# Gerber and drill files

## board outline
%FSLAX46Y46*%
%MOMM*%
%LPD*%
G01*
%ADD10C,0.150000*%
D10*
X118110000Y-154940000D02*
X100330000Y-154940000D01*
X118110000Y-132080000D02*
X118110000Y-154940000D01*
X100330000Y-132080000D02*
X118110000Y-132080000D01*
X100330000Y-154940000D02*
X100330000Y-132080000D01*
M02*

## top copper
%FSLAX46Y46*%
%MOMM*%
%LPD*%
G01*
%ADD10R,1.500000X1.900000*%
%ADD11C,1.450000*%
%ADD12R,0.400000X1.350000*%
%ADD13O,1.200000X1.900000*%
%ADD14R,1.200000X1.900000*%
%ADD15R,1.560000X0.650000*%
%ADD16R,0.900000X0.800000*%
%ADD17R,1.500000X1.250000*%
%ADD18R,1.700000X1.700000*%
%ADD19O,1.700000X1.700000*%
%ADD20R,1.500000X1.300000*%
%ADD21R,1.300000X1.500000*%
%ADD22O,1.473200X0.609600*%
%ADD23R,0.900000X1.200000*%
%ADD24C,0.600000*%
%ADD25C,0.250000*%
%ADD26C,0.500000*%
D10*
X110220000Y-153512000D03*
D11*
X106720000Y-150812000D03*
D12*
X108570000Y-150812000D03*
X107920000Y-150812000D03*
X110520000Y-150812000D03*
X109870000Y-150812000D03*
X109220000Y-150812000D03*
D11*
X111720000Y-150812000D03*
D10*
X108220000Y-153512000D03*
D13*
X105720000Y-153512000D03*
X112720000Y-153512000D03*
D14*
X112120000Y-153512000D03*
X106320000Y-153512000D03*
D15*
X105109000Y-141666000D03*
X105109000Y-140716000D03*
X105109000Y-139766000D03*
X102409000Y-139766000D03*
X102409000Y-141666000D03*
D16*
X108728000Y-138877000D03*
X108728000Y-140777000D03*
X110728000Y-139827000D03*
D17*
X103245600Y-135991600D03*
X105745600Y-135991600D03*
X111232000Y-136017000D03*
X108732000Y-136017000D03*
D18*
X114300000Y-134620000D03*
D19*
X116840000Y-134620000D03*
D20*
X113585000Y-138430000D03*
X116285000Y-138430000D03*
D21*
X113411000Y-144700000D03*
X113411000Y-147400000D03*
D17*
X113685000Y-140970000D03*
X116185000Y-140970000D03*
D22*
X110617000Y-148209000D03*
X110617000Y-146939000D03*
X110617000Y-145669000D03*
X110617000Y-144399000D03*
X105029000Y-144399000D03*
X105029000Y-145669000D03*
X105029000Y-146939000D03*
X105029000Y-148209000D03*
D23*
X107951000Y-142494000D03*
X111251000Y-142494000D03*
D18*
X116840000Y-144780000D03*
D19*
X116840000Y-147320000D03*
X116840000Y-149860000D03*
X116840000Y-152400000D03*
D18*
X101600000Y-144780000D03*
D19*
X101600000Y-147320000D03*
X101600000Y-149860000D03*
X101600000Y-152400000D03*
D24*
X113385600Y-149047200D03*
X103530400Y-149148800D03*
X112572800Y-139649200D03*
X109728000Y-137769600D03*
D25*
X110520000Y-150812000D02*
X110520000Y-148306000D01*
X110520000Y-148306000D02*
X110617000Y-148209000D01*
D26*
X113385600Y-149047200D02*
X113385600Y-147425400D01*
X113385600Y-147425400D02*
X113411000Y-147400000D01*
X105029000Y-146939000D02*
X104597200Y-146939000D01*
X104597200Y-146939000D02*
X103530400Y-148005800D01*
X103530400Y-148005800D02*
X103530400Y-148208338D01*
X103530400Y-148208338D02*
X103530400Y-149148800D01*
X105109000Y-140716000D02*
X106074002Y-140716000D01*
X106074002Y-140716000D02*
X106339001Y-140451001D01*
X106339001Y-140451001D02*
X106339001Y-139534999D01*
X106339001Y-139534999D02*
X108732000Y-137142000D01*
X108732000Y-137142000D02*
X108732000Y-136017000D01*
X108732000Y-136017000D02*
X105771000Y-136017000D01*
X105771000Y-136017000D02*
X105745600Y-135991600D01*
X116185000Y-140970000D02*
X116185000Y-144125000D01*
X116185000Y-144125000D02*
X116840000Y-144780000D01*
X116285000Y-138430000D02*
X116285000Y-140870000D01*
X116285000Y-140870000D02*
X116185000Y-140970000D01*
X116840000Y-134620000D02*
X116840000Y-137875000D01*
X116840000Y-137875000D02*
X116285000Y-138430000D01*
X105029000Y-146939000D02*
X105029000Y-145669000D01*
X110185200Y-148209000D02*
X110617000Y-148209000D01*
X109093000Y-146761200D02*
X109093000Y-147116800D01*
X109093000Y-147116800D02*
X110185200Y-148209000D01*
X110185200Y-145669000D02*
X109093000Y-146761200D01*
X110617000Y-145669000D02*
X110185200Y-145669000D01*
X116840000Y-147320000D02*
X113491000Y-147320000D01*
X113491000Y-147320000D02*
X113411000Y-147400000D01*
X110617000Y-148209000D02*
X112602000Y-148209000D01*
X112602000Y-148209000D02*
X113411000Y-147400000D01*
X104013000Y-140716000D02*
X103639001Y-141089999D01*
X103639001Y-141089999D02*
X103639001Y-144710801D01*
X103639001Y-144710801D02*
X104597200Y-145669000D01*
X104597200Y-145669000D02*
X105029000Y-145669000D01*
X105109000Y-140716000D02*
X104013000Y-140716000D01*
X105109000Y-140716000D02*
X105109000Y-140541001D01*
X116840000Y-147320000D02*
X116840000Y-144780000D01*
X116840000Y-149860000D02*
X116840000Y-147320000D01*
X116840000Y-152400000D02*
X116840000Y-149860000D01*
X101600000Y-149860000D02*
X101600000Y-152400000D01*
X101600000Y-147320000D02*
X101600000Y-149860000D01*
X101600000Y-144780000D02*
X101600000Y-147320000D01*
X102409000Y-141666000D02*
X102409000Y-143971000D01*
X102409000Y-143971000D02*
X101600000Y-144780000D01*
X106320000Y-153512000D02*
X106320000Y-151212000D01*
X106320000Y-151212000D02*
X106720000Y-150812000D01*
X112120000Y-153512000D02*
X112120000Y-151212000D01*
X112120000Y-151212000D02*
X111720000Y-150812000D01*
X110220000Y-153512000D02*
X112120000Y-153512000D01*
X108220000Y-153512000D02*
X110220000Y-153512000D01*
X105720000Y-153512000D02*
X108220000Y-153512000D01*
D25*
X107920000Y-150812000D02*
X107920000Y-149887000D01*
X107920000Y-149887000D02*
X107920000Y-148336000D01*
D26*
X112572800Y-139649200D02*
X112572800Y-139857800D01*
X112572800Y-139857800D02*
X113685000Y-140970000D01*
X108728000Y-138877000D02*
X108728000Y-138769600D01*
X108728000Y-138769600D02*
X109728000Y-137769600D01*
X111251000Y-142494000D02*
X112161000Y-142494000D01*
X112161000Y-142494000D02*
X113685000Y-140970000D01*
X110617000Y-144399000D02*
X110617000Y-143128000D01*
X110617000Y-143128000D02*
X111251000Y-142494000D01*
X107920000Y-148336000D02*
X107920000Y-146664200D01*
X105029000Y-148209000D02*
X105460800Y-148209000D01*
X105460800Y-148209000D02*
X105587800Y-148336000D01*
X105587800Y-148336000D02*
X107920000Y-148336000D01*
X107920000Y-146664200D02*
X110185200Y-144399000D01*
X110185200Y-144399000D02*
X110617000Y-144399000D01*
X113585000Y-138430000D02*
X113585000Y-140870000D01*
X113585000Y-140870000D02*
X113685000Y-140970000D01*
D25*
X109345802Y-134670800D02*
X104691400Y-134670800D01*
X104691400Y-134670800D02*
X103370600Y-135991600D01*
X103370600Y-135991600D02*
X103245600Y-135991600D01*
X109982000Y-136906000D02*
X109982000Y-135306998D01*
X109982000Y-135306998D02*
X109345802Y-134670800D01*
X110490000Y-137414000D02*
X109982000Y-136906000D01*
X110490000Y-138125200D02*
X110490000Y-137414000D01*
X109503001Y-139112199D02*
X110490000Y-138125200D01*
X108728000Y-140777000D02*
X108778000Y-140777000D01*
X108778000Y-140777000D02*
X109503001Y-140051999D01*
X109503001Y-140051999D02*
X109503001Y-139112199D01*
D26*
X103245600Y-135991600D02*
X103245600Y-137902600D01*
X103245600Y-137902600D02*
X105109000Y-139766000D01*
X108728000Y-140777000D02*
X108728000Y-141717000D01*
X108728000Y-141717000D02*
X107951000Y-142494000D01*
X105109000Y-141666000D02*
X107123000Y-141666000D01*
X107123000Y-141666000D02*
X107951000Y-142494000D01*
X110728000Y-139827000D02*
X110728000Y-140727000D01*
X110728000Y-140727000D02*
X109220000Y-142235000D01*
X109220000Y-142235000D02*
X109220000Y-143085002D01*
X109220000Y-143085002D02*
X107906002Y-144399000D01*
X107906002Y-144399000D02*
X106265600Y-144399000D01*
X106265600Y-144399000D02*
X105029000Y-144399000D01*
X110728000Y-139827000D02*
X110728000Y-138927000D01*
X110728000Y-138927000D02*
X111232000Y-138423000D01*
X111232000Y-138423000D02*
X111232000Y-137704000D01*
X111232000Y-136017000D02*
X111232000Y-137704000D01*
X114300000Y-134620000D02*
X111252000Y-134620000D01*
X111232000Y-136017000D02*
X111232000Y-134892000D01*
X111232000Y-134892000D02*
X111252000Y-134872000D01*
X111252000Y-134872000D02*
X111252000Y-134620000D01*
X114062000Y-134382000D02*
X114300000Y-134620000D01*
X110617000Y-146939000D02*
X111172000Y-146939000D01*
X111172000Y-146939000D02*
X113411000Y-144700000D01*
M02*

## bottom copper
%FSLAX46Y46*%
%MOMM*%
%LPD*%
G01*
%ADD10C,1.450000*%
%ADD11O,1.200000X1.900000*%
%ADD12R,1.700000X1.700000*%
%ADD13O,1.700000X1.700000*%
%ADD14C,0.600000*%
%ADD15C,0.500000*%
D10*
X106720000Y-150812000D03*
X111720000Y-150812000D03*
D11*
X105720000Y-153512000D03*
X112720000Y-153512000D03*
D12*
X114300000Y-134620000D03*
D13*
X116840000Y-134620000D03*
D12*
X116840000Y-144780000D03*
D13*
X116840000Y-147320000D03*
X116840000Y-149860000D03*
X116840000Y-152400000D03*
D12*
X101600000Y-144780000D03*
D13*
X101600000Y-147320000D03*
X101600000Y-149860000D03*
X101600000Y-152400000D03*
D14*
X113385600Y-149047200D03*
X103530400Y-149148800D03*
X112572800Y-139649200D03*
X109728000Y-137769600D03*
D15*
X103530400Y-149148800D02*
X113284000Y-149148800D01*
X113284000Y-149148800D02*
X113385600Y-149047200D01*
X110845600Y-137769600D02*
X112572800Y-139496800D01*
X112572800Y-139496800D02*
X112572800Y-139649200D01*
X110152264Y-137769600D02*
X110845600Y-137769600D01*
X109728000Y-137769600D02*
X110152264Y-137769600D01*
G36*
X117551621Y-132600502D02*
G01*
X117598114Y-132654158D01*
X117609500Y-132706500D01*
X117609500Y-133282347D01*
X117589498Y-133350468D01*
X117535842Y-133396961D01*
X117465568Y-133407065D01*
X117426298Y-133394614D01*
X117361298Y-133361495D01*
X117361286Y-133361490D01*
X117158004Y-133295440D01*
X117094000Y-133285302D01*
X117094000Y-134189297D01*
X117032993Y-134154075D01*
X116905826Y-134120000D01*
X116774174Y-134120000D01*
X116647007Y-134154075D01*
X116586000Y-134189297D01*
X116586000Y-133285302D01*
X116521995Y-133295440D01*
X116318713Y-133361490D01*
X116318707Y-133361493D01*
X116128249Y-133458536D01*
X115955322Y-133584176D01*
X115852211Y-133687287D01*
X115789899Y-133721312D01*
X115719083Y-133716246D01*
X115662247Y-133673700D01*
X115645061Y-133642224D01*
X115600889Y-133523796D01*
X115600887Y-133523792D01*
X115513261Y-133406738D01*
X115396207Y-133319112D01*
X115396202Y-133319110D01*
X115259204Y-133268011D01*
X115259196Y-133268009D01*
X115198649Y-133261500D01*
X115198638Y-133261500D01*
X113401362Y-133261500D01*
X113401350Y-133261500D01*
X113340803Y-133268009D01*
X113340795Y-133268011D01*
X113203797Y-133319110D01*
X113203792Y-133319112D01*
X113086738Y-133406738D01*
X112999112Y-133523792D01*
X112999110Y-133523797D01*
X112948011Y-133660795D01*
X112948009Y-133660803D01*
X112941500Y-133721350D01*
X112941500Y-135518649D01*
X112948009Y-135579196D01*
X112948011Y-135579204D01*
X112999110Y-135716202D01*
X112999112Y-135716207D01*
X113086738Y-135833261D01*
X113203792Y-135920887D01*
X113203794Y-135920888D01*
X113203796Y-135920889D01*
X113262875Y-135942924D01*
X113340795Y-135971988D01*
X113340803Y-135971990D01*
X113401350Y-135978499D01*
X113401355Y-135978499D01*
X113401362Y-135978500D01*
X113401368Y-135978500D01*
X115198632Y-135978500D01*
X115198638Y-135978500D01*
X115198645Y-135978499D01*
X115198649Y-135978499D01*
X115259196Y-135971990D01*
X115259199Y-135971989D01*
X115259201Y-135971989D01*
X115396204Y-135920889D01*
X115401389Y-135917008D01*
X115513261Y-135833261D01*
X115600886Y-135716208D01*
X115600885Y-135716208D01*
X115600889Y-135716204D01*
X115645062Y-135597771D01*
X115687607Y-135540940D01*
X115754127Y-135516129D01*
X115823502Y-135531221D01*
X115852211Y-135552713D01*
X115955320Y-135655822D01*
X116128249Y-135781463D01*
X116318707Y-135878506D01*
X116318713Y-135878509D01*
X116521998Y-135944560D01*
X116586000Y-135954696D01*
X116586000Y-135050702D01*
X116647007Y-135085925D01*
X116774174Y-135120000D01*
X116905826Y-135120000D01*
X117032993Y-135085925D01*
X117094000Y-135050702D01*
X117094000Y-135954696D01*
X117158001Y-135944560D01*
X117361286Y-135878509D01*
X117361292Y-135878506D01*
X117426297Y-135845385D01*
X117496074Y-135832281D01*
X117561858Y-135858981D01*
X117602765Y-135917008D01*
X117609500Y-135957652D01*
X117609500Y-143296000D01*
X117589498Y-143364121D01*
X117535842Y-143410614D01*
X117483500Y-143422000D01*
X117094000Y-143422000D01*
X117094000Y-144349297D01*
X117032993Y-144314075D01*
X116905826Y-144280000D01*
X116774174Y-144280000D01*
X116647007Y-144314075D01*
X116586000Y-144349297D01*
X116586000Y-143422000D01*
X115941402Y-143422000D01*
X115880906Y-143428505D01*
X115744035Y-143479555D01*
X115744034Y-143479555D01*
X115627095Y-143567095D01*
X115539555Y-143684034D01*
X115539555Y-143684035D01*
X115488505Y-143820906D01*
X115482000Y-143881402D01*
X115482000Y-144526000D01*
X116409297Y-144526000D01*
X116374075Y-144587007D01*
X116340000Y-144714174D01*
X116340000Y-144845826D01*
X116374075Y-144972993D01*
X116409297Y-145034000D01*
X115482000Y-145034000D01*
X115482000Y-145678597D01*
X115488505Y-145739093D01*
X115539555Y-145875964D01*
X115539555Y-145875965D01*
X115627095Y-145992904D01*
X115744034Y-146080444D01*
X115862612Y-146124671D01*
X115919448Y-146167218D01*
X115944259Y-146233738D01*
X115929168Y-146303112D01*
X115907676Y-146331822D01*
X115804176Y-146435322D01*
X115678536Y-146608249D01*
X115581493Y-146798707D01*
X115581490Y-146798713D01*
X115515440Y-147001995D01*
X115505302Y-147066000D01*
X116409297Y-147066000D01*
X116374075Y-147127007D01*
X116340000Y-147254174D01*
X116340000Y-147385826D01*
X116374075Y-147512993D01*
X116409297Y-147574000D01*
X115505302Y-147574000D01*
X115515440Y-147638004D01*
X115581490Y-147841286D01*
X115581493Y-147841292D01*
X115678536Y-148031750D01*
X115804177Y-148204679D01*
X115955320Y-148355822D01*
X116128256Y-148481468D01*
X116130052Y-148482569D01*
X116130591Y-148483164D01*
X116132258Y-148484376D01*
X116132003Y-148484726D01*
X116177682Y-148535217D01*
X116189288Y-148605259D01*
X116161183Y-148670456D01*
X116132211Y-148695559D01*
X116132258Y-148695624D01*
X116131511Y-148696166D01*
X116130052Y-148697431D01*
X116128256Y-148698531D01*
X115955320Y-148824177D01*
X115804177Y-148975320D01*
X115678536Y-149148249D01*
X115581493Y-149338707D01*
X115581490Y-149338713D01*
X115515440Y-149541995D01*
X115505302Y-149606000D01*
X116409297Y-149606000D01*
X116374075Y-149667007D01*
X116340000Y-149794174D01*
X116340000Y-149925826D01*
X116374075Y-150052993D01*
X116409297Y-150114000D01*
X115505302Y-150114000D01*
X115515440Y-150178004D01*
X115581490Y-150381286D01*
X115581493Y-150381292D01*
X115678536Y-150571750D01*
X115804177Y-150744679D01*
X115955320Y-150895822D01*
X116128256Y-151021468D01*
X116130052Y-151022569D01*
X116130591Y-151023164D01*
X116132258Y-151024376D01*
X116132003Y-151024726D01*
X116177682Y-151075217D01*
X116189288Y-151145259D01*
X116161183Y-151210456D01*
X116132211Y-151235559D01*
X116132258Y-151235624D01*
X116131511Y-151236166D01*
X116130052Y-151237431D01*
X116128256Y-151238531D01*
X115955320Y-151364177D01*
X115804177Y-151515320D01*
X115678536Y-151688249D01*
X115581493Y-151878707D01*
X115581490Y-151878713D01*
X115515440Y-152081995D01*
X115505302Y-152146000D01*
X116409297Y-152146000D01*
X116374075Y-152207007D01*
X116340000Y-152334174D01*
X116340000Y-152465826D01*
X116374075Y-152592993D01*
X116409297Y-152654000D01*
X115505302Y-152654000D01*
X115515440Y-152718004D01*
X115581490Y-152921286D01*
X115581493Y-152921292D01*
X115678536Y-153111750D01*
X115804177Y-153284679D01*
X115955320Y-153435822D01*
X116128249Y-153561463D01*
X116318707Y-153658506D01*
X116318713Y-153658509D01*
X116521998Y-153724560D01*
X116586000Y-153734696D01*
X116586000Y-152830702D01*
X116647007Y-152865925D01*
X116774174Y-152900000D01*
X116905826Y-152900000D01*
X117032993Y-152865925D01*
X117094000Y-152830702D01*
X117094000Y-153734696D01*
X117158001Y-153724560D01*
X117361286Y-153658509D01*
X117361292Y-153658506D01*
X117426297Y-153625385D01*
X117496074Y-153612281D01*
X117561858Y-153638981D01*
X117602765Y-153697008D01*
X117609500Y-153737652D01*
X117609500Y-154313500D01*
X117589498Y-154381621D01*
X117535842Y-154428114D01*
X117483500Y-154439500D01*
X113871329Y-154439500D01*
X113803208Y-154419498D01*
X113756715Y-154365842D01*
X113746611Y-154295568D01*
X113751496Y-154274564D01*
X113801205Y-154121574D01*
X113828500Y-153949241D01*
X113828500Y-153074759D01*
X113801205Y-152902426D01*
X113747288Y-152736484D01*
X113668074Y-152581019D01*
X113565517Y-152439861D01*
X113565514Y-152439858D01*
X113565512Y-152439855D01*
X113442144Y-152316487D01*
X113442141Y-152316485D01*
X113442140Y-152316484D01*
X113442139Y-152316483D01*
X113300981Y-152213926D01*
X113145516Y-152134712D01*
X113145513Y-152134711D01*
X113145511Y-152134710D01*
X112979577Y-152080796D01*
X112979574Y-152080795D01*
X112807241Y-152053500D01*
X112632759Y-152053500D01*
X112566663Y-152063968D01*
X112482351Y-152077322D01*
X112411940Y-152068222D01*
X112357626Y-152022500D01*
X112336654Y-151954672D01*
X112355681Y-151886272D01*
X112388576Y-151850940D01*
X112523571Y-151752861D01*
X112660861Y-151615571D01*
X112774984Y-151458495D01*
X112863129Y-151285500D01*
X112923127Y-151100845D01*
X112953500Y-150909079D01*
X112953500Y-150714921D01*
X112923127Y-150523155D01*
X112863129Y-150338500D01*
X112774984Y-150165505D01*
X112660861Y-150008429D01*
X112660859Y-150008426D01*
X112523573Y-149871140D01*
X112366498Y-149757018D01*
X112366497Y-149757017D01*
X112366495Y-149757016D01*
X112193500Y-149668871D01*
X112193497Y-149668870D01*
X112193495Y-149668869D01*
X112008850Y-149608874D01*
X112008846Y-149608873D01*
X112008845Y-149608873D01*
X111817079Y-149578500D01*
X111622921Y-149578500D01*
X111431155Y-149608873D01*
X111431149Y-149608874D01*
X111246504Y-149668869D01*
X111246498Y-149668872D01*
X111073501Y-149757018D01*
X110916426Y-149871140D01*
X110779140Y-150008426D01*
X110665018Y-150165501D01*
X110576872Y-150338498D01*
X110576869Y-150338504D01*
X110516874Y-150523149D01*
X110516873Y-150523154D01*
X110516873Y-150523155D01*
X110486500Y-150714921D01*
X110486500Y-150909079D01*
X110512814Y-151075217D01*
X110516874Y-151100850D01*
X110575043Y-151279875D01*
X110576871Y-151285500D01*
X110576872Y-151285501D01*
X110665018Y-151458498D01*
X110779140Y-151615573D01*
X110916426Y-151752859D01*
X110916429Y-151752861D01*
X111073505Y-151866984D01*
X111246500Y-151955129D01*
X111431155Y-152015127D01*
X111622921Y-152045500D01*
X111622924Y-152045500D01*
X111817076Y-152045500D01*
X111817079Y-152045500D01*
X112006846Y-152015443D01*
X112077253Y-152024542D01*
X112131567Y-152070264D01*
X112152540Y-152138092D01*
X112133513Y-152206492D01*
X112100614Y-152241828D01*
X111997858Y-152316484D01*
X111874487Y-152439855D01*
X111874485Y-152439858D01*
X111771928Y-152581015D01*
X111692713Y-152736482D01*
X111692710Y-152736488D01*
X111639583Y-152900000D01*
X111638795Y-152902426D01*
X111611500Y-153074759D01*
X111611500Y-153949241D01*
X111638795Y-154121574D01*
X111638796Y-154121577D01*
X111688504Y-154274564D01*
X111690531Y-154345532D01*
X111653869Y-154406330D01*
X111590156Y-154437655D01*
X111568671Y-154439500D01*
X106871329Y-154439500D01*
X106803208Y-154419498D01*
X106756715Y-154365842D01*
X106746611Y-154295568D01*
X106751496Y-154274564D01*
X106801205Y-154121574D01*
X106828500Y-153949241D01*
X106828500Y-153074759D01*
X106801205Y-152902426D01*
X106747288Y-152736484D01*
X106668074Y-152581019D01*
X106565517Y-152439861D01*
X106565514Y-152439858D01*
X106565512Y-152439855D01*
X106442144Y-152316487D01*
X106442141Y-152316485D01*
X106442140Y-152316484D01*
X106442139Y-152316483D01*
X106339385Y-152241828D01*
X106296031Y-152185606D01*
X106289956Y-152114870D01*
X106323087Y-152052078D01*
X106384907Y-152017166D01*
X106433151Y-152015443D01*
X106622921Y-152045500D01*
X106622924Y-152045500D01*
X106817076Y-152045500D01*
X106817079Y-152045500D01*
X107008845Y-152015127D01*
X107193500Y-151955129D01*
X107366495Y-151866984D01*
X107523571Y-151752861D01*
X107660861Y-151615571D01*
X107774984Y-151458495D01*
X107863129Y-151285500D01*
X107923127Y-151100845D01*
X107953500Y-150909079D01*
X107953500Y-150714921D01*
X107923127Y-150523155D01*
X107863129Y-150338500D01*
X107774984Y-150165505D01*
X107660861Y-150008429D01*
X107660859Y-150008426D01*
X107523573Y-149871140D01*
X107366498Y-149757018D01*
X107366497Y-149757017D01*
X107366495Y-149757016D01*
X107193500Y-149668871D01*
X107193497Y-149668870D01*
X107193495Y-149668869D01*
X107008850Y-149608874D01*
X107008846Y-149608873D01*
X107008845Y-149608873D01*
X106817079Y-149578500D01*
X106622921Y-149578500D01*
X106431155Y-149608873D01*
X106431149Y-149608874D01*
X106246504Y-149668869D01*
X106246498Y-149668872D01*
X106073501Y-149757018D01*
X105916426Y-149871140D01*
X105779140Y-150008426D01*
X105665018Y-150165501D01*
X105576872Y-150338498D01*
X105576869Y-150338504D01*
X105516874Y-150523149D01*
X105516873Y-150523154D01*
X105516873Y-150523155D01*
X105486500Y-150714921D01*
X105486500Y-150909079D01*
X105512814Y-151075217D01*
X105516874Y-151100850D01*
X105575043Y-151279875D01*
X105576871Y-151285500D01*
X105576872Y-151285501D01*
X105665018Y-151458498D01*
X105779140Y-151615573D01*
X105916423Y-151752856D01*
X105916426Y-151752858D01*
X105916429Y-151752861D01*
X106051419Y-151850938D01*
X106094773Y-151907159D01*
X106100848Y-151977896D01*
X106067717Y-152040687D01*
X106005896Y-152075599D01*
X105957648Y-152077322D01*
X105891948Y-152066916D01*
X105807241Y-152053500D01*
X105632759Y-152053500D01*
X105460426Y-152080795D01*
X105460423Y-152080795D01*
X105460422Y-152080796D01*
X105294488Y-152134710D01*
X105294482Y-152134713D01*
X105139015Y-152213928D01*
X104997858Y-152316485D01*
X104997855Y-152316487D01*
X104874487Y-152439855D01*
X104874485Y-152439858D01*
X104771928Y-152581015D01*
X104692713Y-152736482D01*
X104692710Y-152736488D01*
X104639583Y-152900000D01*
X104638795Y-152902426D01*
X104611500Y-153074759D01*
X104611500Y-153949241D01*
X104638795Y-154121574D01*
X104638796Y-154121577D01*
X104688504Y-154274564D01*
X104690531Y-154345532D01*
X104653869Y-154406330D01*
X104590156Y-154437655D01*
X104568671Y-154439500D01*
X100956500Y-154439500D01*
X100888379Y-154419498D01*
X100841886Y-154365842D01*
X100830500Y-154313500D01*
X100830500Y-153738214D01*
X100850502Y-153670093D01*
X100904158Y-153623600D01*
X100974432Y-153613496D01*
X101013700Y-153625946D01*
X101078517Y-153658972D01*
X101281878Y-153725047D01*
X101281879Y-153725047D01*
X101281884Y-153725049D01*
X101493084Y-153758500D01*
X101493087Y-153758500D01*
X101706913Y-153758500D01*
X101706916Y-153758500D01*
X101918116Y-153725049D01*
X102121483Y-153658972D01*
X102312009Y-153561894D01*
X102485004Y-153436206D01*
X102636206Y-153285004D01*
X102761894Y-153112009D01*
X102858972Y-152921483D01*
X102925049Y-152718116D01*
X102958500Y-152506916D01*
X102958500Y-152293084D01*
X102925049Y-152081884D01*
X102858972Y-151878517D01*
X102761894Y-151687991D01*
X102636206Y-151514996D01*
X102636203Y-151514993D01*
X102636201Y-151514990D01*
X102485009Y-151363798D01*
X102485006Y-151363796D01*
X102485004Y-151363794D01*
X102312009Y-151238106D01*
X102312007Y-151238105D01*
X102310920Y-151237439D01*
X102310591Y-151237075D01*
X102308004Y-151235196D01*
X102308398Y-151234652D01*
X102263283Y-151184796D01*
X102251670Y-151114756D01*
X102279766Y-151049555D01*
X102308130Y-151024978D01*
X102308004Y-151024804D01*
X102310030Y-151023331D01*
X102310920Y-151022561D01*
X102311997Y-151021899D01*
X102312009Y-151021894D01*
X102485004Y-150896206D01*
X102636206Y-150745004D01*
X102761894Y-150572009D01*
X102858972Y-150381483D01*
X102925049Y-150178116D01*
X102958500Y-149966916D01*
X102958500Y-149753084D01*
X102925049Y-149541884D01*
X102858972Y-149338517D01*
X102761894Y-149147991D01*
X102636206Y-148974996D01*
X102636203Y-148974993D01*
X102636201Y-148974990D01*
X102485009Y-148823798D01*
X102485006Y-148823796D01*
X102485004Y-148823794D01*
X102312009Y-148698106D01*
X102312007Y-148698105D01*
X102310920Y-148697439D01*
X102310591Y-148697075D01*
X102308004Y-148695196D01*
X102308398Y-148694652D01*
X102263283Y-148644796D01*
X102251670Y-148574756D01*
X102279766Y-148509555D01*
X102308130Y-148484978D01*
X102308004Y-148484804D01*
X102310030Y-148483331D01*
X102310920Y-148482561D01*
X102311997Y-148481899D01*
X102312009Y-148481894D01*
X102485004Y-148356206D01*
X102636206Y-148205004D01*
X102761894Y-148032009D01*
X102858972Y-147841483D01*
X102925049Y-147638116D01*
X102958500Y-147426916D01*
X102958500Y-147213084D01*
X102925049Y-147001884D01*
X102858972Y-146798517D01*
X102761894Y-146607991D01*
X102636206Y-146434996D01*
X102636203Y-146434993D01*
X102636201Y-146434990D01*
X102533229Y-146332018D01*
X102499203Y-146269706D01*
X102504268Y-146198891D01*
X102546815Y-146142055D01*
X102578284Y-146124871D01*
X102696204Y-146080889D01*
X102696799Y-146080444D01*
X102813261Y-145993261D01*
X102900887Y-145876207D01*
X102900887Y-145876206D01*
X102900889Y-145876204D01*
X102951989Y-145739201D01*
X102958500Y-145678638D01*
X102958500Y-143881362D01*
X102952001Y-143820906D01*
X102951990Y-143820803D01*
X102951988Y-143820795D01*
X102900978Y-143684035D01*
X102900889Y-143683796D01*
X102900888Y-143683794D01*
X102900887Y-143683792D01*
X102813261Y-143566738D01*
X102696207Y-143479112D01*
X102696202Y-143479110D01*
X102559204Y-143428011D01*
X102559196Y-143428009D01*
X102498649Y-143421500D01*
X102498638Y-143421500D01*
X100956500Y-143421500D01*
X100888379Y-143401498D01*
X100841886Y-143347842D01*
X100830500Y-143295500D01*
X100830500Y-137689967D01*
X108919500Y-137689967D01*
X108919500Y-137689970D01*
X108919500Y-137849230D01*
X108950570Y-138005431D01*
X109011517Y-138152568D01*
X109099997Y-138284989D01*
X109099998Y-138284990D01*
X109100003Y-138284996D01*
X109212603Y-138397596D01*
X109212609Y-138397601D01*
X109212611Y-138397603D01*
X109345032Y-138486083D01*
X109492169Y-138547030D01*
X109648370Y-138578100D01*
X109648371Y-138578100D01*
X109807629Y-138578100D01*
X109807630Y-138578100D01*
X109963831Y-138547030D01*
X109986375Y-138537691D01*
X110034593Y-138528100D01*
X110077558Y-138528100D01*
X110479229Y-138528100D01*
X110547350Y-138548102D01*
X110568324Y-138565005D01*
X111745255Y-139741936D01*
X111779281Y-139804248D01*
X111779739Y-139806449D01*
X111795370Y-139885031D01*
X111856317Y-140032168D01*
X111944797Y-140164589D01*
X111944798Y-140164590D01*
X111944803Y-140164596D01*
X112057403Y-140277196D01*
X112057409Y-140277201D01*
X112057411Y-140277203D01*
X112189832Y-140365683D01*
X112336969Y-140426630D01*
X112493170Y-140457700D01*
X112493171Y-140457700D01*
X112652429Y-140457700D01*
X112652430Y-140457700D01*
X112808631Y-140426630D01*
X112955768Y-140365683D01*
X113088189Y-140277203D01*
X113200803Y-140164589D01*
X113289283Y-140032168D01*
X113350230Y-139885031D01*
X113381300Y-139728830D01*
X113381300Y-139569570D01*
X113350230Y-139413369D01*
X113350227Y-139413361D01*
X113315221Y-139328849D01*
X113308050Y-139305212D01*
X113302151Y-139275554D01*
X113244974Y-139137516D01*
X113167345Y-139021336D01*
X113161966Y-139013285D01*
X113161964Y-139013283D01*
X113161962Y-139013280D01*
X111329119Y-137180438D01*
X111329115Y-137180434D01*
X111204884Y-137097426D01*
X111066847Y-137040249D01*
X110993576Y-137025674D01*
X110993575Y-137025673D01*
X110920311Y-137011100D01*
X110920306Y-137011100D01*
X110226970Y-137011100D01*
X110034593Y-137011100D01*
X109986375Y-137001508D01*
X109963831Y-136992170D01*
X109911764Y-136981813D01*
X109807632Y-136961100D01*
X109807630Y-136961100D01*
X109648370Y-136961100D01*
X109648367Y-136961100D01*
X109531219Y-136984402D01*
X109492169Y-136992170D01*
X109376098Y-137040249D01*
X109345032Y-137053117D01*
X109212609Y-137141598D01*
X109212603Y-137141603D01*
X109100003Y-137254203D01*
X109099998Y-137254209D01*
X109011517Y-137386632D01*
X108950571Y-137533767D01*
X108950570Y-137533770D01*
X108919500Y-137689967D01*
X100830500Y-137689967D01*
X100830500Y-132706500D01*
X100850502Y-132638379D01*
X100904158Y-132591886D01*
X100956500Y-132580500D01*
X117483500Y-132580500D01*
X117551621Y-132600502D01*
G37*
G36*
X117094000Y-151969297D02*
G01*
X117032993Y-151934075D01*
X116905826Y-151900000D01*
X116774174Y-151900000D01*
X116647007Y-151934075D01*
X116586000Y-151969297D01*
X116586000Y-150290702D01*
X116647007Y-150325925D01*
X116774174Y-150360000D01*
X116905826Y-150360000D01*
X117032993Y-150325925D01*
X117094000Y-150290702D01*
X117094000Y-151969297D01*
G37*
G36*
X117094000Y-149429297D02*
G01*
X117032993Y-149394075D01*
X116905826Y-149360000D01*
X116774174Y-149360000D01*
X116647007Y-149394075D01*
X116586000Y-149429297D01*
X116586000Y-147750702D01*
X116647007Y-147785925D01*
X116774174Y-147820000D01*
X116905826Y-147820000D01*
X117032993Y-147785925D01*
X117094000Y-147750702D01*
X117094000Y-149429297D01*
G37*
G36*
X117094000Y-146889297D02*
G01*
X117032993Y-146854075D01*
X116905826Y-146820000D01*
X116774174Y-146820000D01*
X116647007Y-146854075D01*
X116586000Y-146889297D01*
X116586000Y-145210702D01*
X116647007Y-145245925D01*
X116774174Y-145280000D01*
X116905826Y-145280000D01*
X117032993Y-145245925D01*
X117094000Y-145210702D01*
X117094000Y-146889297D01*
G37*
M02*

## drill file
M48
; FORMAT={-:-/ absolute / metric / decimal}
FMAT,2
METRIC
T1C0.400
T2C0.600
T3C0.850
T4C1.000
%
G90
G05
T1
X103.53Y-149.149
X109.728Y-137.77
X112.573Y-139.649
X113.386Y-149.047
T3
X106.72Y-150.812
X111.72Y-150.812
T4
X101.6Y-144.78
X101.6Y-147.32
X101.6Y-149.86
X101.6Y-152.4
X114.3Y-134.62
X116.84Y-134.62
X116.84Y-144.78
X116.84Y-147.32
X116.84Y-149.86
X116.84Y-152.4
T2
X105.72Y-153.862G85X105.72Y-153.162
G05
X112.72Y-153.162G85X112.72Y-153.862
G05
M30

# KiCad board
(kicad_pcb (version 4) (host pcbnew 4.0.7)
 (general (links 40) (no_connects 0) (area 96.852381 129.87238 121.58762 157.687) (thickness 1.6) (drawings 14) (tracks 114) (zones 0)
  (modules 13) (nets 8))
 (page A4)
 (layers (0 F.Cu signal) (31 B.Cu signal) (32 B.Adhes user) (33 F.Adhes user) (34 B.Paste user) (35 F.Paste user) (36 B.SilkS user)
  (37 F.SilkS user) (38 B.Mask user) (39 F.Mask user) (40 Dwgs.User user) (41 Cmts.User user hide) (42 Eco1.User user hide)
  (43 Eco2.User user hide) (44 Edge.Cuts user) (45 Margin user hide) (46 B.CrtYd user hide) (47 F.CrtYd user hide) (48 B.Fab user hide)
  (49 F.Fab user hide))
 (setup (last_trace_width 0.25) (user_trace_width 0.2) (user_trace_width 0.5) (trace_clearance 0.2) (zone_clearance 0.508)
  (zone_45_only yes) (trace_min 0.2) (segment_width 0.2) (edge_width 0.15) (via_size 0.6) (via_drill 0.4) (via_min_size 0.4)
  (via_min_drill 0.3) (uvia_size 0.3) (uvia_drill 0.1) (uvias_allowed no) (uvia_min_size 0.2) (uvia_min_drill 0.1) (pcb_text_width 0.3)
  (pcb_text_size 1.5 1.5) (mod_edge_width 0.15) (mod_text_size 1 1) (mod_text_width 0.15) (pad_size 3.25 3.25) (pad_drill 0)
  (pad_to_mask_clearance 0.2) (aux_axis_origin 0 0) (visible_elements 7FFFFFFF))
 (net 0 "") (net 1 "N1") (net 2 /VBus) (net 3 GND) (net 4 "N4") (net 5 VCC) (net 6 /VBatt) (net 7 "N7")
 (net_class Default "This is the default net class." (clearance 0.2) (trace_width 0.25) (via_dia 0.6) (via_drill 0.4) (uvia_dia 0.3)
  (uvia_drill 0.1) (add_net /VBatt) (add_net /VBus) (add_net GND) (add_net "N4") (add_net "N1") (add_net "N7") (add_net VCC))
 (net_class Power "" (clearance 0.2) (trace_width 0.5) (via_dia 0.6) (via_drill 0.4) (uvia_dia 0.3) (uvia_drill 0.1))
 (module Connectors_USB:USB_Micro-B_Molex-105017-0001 (layer F.Cu) (at 109.22 153.162)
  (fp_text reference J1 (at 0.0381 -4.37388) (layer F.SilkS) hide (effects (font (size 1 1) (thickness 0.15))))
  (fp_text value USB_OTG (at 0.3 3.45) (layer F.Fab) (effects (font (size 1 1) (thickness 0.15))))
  (pad 6 smd rect (at 1 0.35) (size 1.5 1.9) (layers F.Cu F.Paste F.Mask) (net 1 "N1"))
  (pad 6 thru_hole circle (at -2.5 -2.35) (size 1.45 1.45) (drill 0.85) (layers *.Cu *.Mask) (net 1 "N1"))
  (pad 2 smd rect (at -0.65 -2.35) (size 0.4 1.35) (layers F.Cu F.Paste F.Mask))
  (pad 1 smd rect (at -1.3 -2.35) (size 0.4 1.35) (layers F.Cu F.Paste F.Mask) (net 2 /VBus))
  (pad 5 smd rect (at 1.3 -2.35) (size 0.4 1.35) (layers F.Cu F.Paste F.Mask) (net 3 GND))
  (pad 4 smd rect (at 0.65 -2.35) (size 0.4 1.35) (layers F.Cu F.Paste F.Mask))
  (pad 3 smd rect (at 0 -2.35) (size 0.4 1.35) (layers F.Cu F.Paste F.Mask))
  (pad 6 thru_hole circle (at 2.5 -2.35) (size 1.45 1.45) (drill 0.85) (layers *.Cu *.Mask) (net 1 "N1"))
  (pad 6 smd rect (at -1 0.35) (size 1.5 1.9) (layers F.Cu F.Paste F.Mask) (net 1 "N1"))
  (pad 6 thru_hole oval (at -3.5 0.35 180) (size 1.2 1.9) (drill oval 0.6 1.3) (layers *.Cu *.Mask) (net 1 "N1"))
  (pad 6 thru_hole oval (at 3.5 0.35) (size 1.2 1.9) (drill oval 0.6 1.3) (layers *.Cu *.Mask) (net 1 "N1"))
  (pad 6 smd rect (at 2.9 0.35) (size 1.2 1.9) (layers F.Cu F.Mask) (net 1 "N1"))
  (pad 6 smd rect (at -2.9 0.35) (size 1.2 1.9) (layers F.Cu F.Mask) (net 1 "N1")))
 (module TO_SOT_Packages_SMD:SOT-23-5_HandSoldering (layer F.Cu) (at 103.759 140.716 180)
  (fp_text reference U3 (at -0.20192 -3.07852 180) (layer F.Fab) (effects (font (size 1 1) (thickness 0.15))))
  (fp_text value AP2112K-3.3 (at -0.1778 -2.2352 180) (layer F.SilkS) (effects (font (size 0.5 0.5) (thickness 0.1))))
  (pad 1 smd rect (at -1.35 -0.95 180) (size 1.56 0.65) (layers F.Cu F.Paste F.Mask) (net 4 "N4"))
  (pad 2 smd rect (at -1.35 0 180) (size 1.56 0.65) (layers F.Cu F.Paste F.Mask) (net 3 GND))
  (pad 3 smd rect (at -1.35 0.95 180) (size 1.56 0.65) (layers F.Cu F.Paste F.Mask) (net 4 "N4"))
  (pad 4 smd rect (at 1.35 0.95 180) (size 1.56 0.65) (layers F.Cu F.Paste F.Mask))
  (pad 5 smd rect (at 1.35 -0.95 180) (size 1.56 0.65) (layers F.Cu F.Paste F.Mask) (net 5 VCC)))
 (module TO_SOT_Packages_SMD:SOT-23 (layer F.Cu) (at 109.728 139.827)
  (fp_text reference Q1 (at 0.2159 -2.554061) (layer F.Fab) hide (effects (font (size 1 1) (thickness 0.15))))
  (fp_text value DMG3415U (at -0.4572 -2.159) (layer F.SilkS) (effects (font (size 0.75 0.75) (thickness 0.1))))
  (pad 1 smd rect (at -1 -0.95) (size 0.9 0.8) (layers F.Cu F.Paste F.Mask) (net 2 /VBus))
  (pad 2 smd rect (at -1 0.95) (size 0.9 0.8) (layers F.Cu F.Paste F.Mask) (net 4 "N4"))
  (pad 3 smd rect (at 1 0) (size 0.9 0.8) (layers F.Cu F.Paste F.Mask) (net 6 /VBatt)))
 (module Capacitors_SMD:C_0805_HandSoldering (layer F.Cu) (at 104.4956 135.9916)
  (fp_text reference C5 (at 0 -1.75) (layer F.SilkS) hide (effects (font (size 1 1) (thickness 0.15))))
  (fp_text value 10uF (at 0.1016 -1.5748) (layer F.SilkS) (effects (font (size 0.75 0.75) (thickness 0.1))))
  (pad 1 smd rect (at -1.25 0) (size 1.5 1.25) (layers F.Cu F.Paste F.Mask) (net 4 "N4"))
  (pad 2 smd rect (at 1.25 0) (size 1.5 1.25) (layers F.Cu F.Paste F.Mask) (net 3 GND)))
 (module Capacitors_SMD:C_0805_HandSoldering (layer F.Cu) (at 109.982 136.017 180)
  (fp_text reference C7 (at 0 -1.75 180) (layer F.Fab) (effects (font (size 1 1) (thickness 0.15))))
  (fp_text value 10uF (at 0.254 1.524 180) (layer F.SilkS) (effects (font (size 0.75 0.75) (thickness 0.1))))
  (pad 1 smd rect (at -1.25 0 180) (size 1.5 1.25) (layers F.Cu F.Paste F.Mask) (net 6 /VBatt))
  (pad 2 smd rect (at 1.25 0 180) (size 1.5 1.25) (layers F.Cu F.Paste F.Mask) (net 3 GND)))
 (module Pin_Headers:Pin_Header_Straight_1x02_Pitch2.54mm (layer F.Cu) (at 114.3 134.62 90)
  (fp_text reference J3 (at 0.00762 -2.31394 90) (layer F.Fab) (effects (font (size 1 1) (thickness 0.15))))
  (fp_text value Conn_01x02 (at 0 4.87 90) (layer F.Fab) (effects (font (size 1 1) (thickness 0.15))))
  (pad 1 thru_hole rect (at 0 0 90) (size 1.7 1.7) (drill 1) (layers *.Cu *.Mask) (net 6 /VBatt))
  (pad 2 thru_hole oval (at 0 2.54 90) (size 1.7 1.7) (drill 1) (layers *.Cu *.Mask) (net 3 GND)))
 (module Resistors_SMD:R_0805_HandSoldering (layer F.Cu) (at 114.935 138.43)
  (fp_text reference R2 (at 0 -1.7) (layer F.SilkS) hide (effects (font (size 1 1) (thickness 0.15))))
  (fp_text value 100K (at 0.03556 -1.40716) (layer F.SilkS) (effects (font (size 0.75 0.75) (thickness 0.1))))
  (pad 1 smd rect (at -1.35 0) (size 1.5 1.3) (layers F.Cu F.Paste F.Mask) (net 2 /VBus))
  (pad 2 smd rect (at 1.35 0) (size 1.5 1.3) (layers F.Cu F.Paste F.Mask) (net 3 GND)))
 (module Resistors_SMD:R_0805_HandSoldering (layer F.Cu) (at 113.411 146.05 270)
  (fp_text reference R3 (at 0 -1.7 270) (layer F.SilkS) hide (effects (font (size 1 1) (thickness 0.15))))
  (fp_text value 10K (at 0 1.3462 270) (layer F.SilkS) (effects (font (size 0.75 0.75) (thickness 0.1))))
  (pad 1 smd rect (at -1.35 0 270) (size 1.5 1.3) (layers F.Cu F.Paste F.Mask) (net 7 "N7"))
  (pad 2 smd rect (at 1.35 0 270) (size 1.5 1.3) (layers F.Cu F.Paste F.Mask) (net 3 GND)))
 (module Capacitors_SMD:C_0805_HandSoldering (layer F.Cu) (at 114.935 140.97)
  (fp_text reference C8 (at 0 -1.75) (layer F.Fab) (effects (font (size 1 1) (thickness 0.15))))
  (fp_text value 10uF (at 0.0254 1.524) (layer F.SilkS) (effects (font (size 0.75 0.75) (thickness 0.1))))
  (pad 1 smd rect (at -1.25 0) (size 1.5 1.25) (layers F.Cu F.Paste F.Mask) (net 2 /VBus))
  (pad 2 smd rect (at 1.25 0) (size 1.5 1.25) (layers F.Cu F.Paste F.Mask) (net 3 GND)))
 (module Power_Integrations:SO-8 (layer F.Cu) (at 107.823 146.304 90)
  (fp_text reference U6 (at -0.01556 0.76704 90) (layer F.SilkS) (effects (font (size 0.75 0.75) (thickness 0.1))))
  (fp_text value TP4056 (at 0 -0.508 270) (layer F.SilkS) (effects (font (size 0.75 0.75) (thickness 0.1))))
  (pad 1 smd oval (at -1.905 2.794 90) (size 0.6096 1.4732) (layers F.Cu F.Paste F.Mask) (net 3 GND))
  (pad 2 smd oval (at -0.635 2.794 90) (size 0.6096 1.4732) (layers F.Cu F.Paste F.Mask) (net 7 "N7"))
  (pad 3 smd oval (at 0.635 2.794 90) (size 0.6096 1.4732) (layers F.Cu F.Paste F.Mask) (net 3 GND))
  (pad 4 smd oval (at 1.905 2.794 90) (size 0.6096 1.4732) (layers F.Cu F.Paste F.Mask) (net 2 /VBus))
  (pad 5 smd oval (at 1.905 -2.794 90) (size 0.6096 1.4732) (layers F.Cu F.Paste F.Mask) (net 6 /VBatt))
  (pad 6 smd oval (at 0.635 -2.794 90) (size 0.6096 1.4732) (layers F.Cu F.Paste F.Mask) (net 3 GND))
  (pad 7 smd oval (at -0.635 -2.794 90) (size 0.6096 1.4732) (layers F.Cu F.Paste F.Mask) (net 3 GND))
  (pad 8 smd oval (at -1.905 -2.794 90) (size 0.6096 1.4732) (layers F.Cu F.Paste F.Mask) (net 2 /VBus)))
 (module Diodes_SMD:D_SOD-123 (layer F.Cu) (at 109.601 142.494)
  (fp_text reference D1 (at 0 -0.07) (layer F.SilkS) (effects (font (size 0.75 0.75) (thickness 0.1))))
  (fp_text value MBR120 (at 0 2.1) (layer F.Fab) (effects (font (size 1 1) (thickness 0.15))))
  (pad 1 smd rect (at -1.65 0) (size 0.9 1.2) (layers F.Cu F.Paste F.Mask) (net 4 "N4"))
  (pad 2 smd rect (at 1.65 0) (size 0.9 1.2) (layers F.Cu F.Paste F.Mask) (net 2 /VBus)))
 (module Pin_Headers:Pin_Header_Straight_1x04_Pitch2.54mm (layer F.Cu) (at 116.84 144.78)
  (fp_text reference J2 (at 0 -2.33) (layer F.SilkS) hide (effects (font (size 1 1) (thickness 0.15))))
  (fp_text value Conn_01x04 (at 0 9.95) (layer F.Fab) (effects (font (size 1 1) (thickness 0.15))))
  (pad 1 thru_hole rect (at 0 0) (size 1.7 1.7) (drill 1) (layers *.Cu *.Mask) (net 3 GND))
  (pad 2 thru_hole oval (at 0 2.54) (size 1.7 1.7) (drill 1) (layers *.Cu *.Mask) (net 3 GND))
  (pad 3 thru_hole oval (at 0 5.08) (size 1.7 1.7) (drill 1) (layers *.Cu *.Mask) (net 3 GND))
  (pad 4 thru_hole oval (at 0 7.62) (size 1.7 1.7) (drill 1) (layers *.Cu *.Mask) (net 3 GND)))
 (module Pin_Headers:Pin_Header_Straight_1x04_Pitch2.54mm (layer F.Cu) (at 101.6 144.78)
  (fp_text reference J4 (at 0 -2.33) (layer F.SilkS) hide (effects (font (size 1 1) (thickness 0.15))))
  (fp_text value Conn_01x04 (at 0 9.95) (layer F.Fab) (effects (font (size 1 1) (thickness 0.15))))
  (pad 1 thru_hole rect (at 0 0) (size 1.7 1.7) (drill 1) (layers *.Cu *.Mask) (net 5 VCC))
  (pad 2 thru_hole oval (at 0 2.54) (size 1.7 1.7) (drill 1) (layers *.Cu *.Mask) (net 5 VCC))
  (pad 3 thru_hole oval (at 0 5.08) (size 1.7 1.7) (drill 1) (layers *.Cu *.Mask) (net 5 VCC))
  (pad 4 thru_hole oval (at 0 7.62) (size 1.7 1.7) (drill 1) (layers *.Cu *.Mask) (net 5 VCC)))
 (gr_line (start 118.11 154.94) (end 100.33 154.94) (layer Edge.Cuts) (width 0.15))
 (gr_line (start 118.11 132.08) (end 118.11 154.94) (layer Edge.Cuts) (width 0.15))
 (gr_line (start 100.33 132.08) (end 118.11 132.08) (layer Edge.Cuts) (width 0.15))
 (gr_line (start 100.33 154.94) (end 100.33 132.08) (layer Edge.Cuts) (width 0.15))
 (segment (start 110.52 150.812) (end 110.52 148.306) (width 0.25) (layer F.Cu) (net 3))
 (segment (start 110.52 148.306) (end 110.617 148.209) (width 0.25) (layer F.Cu) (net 3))
 (segment (start 113.3856 149.0472) (end 113.3856 147.4254) (width 0.5) (layer F.Cu) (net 3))
 (segment (start 113.3856 147.4254) (end 113.411 147.4) (width 0.5) (layer F.Cu) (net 3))
 (segment (start 103.5304 149.1488) (end 113.284 149.1488) (width 0.5) (layer B.Cu) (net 3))
 (segment (start 113.284 149.1488) (end 113.3856 149.0472) (width 0.5) (layer B.Cu) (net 3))
 (via (at 113.3856 149.0472) (size 0.6) (drill 0.4) (layers F.Cu B.Cu) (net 3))
 (segment (start 105.029 146.939) (end 104.5972 146.939) (width 0.5) (layer F.Cu) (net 3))
 (segment (start 104.5972 146.939) (end 103.5304 148.0058) (width 0.5) (layer F.Cu) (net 3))
 (segment (start 103.5304 148.0058) (end 103.5304 148.208338) (width 0.5) (layer F.Cu) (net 3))
 (segment (start 103.5304 148.208338) (end 103.5304 149.1488) (width 0.5) (layer F.Cu) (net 3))
 (via (at 103.5304 149.1488) (size 0.6) (drill 0.4) (layers F.Cu B.Cu) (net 3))
 (segment (start 105.109 140.716) (end 106.074002 140.716) (width 0.5) (layer F.Cu) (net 3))
 (segment (start 106.074002 140.716) (end 106.339001 140.451001) (width 0.5) (layer F.Cu) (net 3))
 (segment (start 106.339001 140.451001) (end 106.339001 139.534999) (width 0.5) (layer F.Cu) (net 3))
 (segment (start 106.339001 139.534999) (end 108.732 137.142) (width 0.5) (layer F.Cu) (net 3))
 (segment (start 108.732 137.142) (end 108.732 136.017) (width 0.5) (layer F.Cu) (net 3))
 (segment (start 108.732 136.017) (end 105.771 136.017) (width 0.5) (layer F.Cu) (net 3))
 (segment (start 105.771 136.017) (end 105.7456 135.9916) (width 0.5) (layer F.Cu) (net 3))
 (segment (start 116.185 140.97) (end 116.185 144.125) (width 0.5) (layer F.Cu) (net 3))
 (segment (start 116.185 144.125) (end 116.84 144.78) (width 0.5) (layer F.Cu) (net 3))
 (segment (start 116.285 138.43) (end 116.285 140.87) (width 0.5) (layer F.Cu) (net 3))
 (segment (start 116.285 140.87) (end 116.185 140.97) (width 0.5) (layer F.Cu) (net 3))
 (segment (start 116.84 134.62) (end 116.84 137.875) (width 0.5) (layer F.Cu) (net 3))
 (segment (start 116.84 137.875) (end 116.285 138.43) (width 0.5) (layer F.Cu) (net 3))
 (segment (start 105.029 146.939) (end 105.029 145.669) (width 0.5) (layer F.Cu) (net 3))
 (segment (start 110.1852 148.209) (end 110.617 148.209) (width 0.5) (layer F.Cu) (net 3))
 (segment (start 109.093 146.7612) (end 109.093 147.1168) (width 0.5) (layer F.Cu) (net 3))
 (segment (start 109.093 147.1168) (end 110.1852 148.209) (width 0.5) (layer F.Cu) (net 3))
 (segment (start 110.1852 145.669) (end 109.093 146.7612) (width 0.5) (layer F.Cu) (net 3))
 (segment (start 110.617 145.669) (end 110.1852 145.669) (width 0.5) (layer F.Cu) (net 3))
 (segment (start 116.84 147.32) (end 113.491 147.32) (width 0.5) (layer F.Cu) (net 3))
 (segment (start 113.491 147.32) (end 113.411 147.4) (width 0.5) (layer F.Cu) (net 3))
 (segment (start 110.617 148.209) (end 112.602 148.209) (width 0.5) (layer F.Cu) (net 3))
 (segment (start 112.602 148.209) (end 113.411 147.4) (width 0.5) (layer F.Cu) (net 3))
 (segment (start 104.013 140.716) (end 103.639001 141.089999) (width 0.5) (layer F.Cu) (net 3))
 (segment (start 103.639001 141.089999) (end 103.639001 144.710801) (width 0.5) (layer F.Cu) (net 3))
 (segment (start 103.639001 144.710801) (end 104.5972 145.669) (width 0.5) (layer F.Cu) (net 3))
 (segment (start 104.5972 145.669) (end 105.029 145.669) (width 0.5) (layer F.Cu) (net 3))
 (segment (start 105.109 140.716) (end 104.013 140.716) (width 0.5) (layer F.Cu) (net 3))
 (segment (start 105.109 140.716) (end 105.109 140.541001) (width 0.5) (layer F.Cu) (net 3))
 (segment (start 116.84 147.32) (end 116.84 144.78) (width 0.5) (layer F.Cu) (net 3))
 (segment (start 116.84 149.86) (end 116.84 147.32) (width 0.5) (layer F.Cu) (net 3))
 (segment (start 116.84 152.4) (end 116.84 149.86) (width 0.5) (layer F.Cu) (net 3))
 (segment (start 101.6 149.86) (end 101.6 152.4) (width 0.5) (layer F.Cu) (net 5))
 (segment (start 101.6 147.32) (end 101.6 149.86) (width 0.5) (layer F.Cu) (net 5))
 (segment (start 101.6 144.78) (end 101.6 147.32) (width 0.5) (layer F.Cu) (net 5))
 (segment (start 102.409 141.666) (end 102.409 143.971) (width 0.5) (layer F.Cu) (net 5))
 (segment (start 102.409 143.971) (end 101.6 144.78) (width 0.5) (layer F.Cu) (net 5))
 (segment (start 106.32 153.512) (end 106.32 151.212) (width 0.5) (layer F.Cu) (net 1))
 (segment (start 106.32 151.212) (end 106.72 150.812) (width 0.5) (layer F.Cu) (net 1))
 (segment (start 112.12 153.512) (end 112.12 151.212) (width 0.5) (layer F.Cu) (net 1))
 (segment (start 112.12 151.212) (end 111.72 150.812) (width 0.5) (layer F.Cu) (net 1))
 (segment (start 110.22 153.512) (end 112.12 153.512) (width 0.5) (layer F.Cu) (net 1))
 (segment (start 108.22 153.512) (end 110.22 153.512) (width 0.5) (layer F.Cu) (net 1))
 (segment (start 105.72 153.512) (end 108.22 153.512) (width 0.5) (layer F.Cu) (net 1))
 (segment (start 107.92 150.812) (end 107.92 149.887) (width 0.25) (layer F.Cu) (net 2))
 (segment (start 107.92 149.887) (end 107.92 148.336) (width 0.25) (layer F.Cu) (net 2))
 (segment (start 112.5728 139.6492) (end 112.5728 139.8578) (width 0.5) (layer F.Cu) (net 2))
 (segment (start 112.5728 139.8578) (end 113.685 140.97) (width 0.5) (layer F.Cu) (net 2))
 (segment (start 110.8456 137.7696) (end 112.5728 139.4968) (width 0.5) (layer B.Cu) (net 2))
 (segment (start 112.5728 139.4968) (end 112.5728 139.6492) (width 0.5) (layer B.Cu) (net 2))
 (via (at 112.5728 139.6492) (size 0.6) (drill 0.4) (layers F.Cu B.Cu) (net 2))
 (segment (start 110.152264 137.7696) (end 110.8456 137.7696) (width 0.5) (layer B.Cu) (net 2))
 (segment (start 109.728 137.7696) (end 110.152264 137.7696) (width 0.5) (layer B.Cu) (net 2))
 (segment (start 108.728 138.877) (end 108.728 138.7696) (width 0.5) (layer F.Cu) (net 2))
 (segment (start 108.728 138.7696) (end 109.728 137.7696) (width 0.5) (layer F.Cu) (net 2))
 (via (at 109.728 137.7696) (size 0.6) (drill 0.4) (layers F.Cu B.Cu) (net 2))
 (segment (start 111.251 142.494) (end 112.161 142.494) (width 0.5) (layer F.Cu) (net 2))
 (segment (start 112.161 142.494) (end 113.685 140.97) (width 0.5) (layer F.Cu) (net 2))
 (segment (start 110.617 144.399) (end 110.617 143.128) (width 0.5) (layer F.Cu) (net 2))
 (segment (start 110.617 143.128) (end 111.251 142.494) (width 0.5) (layer F.Cu) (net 2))
 (segment (start 107.92 148.336) (end 107.92 146.6642) (width 0.5) (layer F.Cu) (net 2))
 (segment (start 105.029 148.209) (end 105.4608 148.209) (width 0.5) (layer F.Cu) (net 2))
 (segment (start 105.4608 148.209) (end 105.5878 148.336) (width 0.5) (layer F.Cu) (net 2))
 (segment (start 105.5878 148.336) (end 107.92 148.336) (width 0.5) (layer F.Cu) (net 2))
 (segment (start 107.92 146.6642) (end 110.1852 144.399) (width 0.5) (layer F.Cu) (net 2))
 (segment (start 110.1852 144.399) (end 110.617 144.399) (width 0.5) (layer F.Cu) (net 2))
 (segment (start 113.585 138.43) (end 113.585 140.87) (width 0.5) (layer F.Cu) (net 2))
 (segment (start 113.585 140.87) (end 113.685 140.97) (width 0.5) (layer F.Cu) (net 2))
 (segment (start 109.345802 134.6708) (end 104.6914 134.6708) (width 0.25) (layer F.Cu) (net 4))
 (segment (start 104.6914 134.6708) (end 103.3706 135.9916) (width 0.25) (layer F.Cu) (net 4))
 (segment (start 103.3706 135.9916) (end 103.2456 135.9916) (width 0.25) (layer F.Cu) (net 4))
 (segment (start 109.982 136.906) (end 109.982 135.306998) (width 0.25) (layer F.Cu) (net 4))
 (segment (start 109.982 135.306998) (end 109.345802 134.6708) (width 0.25) (layer F.Cu) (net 4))
 (segment (start 110.49 137.414) (end 109.982 136.906) (width 0.25) (layer F.Cu) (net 4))
 (segment (start 110.49 138.1252) (end 110.49 137.414) (width 0.25) (layer F.Cu) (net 4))
 (segment (start 109.503001 139.112199) (end 110.49 138.1252) (width 0.25) (layer F.Cu) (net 4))
 (segment (start 108.728 140.777) (end 108.778 140.777) (width 0.25) (layer F.Cu) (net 4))
 (segment (start 108.778 140.777) (end 109.503001 140.051999) (width 0.25) (layer F.Cu) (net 4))
 (segment (start 109.503001 140.051999) (end 109.503001 139.112199) (width 0.25) (layer F.Cu) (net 4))
 (segment (start 103.2456 135.9916) (end 103.2456 137.9026) (width 0.5) (layer F.Cu) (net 4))
 (segment (start 103.2456 137.9026) (end 105.109 139.766) (width 0.5) (layer F.Cu) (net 4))
 (segment (start 108.728 140.777) (end 108.728 141.717) (width 0.5) (layer F.Cu) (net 4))
 (segment (start 108.728 141.717) (end 107.951 142.494) (width 0.5) (layer F.Cu) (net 4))
 (segment (start 105.109 141.666) (end 107.123 141.666) (width 0.5) (layer F.Cu) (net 4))
 (segment (start 107.123 141.666) (end 107.951 142.494) (width 0.5) (layer F.Cu) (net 4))
 (segment (start 110.728 139.827) (end 110.728 140.727) (width 0.5) (layer F.Cu) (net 6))
 (segment (start 110.728 140.727) (end 109.22 142.235) (width 0.5) (layer F.Cu) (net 6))
 (segment (start 109.22 142.235) (end 109.22 143.085002) (width 0.5) (layer F.Cu) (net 6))
 (segment (start 109.22 143.085002) (end 107.906002 144.399) (width 0.5) (layer F.Cu) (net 6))
 (segment (start 107.906002 144.399) (end 106.2656 144.399) (width 0.5) (layer F.Cu) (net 6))
 (segment (start 106.2656 144.399) (end 105.029 144.399) (width 0.5) (layer F.Cu) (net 6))
 (segment (start 110.728 139.827) (end 110.728 138.927) (width 0.5) (layer F.Cu) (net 6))
 (segment (start 110.728 138.927) (end 111.232 138.423) (width 0.5) (layer F.Cu) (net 6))
 (segment (start 111.232 138.423) (end 111.232 137.704) (width 0.5) (layer F.Cu) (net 6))
 (segment (start 111.232 136.017) (end 111.232 137.704) (width 0.5) (layer F.Cu) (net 6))
 (segment (start 114.3 134.62) (end 111.252 134.62) (width 0.5) (layer F.Cu) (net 6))
 (segment (start 111.232 136.017) (end 111.232 134.892) (width 0.5) (layer F.Cu) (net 6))
 (segment (start 111.232 134.892) (end 111.252 134.872) (width 0.5) (layer F.Cu) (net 6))
 (segment (start 111.252 134.872) (end 111.252 134.62) (width 0.5) (layer F.Cu) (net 6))
 (segment (start 114.062 134.382) (end 114.3 134.62) (width 0.5) (layer F.Cu) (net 6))
 (segment (start 110.617 146.939) (end 111.172 146.939) (width 0.5) (layer F.Cu) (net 7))
 (segment (start 111.172 146.939) (end 113.411 144.7) (width 0.5) (layer F.Cu) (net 7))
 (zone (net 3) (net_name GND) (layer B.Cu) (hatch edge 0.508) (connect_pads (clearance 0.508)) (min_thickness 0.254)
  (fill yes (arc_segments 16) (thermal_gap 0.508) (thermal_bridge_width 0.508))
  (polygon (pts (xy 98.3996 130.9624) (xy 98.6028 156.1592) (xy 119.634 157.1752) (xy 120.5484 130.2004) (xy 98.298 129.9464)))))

